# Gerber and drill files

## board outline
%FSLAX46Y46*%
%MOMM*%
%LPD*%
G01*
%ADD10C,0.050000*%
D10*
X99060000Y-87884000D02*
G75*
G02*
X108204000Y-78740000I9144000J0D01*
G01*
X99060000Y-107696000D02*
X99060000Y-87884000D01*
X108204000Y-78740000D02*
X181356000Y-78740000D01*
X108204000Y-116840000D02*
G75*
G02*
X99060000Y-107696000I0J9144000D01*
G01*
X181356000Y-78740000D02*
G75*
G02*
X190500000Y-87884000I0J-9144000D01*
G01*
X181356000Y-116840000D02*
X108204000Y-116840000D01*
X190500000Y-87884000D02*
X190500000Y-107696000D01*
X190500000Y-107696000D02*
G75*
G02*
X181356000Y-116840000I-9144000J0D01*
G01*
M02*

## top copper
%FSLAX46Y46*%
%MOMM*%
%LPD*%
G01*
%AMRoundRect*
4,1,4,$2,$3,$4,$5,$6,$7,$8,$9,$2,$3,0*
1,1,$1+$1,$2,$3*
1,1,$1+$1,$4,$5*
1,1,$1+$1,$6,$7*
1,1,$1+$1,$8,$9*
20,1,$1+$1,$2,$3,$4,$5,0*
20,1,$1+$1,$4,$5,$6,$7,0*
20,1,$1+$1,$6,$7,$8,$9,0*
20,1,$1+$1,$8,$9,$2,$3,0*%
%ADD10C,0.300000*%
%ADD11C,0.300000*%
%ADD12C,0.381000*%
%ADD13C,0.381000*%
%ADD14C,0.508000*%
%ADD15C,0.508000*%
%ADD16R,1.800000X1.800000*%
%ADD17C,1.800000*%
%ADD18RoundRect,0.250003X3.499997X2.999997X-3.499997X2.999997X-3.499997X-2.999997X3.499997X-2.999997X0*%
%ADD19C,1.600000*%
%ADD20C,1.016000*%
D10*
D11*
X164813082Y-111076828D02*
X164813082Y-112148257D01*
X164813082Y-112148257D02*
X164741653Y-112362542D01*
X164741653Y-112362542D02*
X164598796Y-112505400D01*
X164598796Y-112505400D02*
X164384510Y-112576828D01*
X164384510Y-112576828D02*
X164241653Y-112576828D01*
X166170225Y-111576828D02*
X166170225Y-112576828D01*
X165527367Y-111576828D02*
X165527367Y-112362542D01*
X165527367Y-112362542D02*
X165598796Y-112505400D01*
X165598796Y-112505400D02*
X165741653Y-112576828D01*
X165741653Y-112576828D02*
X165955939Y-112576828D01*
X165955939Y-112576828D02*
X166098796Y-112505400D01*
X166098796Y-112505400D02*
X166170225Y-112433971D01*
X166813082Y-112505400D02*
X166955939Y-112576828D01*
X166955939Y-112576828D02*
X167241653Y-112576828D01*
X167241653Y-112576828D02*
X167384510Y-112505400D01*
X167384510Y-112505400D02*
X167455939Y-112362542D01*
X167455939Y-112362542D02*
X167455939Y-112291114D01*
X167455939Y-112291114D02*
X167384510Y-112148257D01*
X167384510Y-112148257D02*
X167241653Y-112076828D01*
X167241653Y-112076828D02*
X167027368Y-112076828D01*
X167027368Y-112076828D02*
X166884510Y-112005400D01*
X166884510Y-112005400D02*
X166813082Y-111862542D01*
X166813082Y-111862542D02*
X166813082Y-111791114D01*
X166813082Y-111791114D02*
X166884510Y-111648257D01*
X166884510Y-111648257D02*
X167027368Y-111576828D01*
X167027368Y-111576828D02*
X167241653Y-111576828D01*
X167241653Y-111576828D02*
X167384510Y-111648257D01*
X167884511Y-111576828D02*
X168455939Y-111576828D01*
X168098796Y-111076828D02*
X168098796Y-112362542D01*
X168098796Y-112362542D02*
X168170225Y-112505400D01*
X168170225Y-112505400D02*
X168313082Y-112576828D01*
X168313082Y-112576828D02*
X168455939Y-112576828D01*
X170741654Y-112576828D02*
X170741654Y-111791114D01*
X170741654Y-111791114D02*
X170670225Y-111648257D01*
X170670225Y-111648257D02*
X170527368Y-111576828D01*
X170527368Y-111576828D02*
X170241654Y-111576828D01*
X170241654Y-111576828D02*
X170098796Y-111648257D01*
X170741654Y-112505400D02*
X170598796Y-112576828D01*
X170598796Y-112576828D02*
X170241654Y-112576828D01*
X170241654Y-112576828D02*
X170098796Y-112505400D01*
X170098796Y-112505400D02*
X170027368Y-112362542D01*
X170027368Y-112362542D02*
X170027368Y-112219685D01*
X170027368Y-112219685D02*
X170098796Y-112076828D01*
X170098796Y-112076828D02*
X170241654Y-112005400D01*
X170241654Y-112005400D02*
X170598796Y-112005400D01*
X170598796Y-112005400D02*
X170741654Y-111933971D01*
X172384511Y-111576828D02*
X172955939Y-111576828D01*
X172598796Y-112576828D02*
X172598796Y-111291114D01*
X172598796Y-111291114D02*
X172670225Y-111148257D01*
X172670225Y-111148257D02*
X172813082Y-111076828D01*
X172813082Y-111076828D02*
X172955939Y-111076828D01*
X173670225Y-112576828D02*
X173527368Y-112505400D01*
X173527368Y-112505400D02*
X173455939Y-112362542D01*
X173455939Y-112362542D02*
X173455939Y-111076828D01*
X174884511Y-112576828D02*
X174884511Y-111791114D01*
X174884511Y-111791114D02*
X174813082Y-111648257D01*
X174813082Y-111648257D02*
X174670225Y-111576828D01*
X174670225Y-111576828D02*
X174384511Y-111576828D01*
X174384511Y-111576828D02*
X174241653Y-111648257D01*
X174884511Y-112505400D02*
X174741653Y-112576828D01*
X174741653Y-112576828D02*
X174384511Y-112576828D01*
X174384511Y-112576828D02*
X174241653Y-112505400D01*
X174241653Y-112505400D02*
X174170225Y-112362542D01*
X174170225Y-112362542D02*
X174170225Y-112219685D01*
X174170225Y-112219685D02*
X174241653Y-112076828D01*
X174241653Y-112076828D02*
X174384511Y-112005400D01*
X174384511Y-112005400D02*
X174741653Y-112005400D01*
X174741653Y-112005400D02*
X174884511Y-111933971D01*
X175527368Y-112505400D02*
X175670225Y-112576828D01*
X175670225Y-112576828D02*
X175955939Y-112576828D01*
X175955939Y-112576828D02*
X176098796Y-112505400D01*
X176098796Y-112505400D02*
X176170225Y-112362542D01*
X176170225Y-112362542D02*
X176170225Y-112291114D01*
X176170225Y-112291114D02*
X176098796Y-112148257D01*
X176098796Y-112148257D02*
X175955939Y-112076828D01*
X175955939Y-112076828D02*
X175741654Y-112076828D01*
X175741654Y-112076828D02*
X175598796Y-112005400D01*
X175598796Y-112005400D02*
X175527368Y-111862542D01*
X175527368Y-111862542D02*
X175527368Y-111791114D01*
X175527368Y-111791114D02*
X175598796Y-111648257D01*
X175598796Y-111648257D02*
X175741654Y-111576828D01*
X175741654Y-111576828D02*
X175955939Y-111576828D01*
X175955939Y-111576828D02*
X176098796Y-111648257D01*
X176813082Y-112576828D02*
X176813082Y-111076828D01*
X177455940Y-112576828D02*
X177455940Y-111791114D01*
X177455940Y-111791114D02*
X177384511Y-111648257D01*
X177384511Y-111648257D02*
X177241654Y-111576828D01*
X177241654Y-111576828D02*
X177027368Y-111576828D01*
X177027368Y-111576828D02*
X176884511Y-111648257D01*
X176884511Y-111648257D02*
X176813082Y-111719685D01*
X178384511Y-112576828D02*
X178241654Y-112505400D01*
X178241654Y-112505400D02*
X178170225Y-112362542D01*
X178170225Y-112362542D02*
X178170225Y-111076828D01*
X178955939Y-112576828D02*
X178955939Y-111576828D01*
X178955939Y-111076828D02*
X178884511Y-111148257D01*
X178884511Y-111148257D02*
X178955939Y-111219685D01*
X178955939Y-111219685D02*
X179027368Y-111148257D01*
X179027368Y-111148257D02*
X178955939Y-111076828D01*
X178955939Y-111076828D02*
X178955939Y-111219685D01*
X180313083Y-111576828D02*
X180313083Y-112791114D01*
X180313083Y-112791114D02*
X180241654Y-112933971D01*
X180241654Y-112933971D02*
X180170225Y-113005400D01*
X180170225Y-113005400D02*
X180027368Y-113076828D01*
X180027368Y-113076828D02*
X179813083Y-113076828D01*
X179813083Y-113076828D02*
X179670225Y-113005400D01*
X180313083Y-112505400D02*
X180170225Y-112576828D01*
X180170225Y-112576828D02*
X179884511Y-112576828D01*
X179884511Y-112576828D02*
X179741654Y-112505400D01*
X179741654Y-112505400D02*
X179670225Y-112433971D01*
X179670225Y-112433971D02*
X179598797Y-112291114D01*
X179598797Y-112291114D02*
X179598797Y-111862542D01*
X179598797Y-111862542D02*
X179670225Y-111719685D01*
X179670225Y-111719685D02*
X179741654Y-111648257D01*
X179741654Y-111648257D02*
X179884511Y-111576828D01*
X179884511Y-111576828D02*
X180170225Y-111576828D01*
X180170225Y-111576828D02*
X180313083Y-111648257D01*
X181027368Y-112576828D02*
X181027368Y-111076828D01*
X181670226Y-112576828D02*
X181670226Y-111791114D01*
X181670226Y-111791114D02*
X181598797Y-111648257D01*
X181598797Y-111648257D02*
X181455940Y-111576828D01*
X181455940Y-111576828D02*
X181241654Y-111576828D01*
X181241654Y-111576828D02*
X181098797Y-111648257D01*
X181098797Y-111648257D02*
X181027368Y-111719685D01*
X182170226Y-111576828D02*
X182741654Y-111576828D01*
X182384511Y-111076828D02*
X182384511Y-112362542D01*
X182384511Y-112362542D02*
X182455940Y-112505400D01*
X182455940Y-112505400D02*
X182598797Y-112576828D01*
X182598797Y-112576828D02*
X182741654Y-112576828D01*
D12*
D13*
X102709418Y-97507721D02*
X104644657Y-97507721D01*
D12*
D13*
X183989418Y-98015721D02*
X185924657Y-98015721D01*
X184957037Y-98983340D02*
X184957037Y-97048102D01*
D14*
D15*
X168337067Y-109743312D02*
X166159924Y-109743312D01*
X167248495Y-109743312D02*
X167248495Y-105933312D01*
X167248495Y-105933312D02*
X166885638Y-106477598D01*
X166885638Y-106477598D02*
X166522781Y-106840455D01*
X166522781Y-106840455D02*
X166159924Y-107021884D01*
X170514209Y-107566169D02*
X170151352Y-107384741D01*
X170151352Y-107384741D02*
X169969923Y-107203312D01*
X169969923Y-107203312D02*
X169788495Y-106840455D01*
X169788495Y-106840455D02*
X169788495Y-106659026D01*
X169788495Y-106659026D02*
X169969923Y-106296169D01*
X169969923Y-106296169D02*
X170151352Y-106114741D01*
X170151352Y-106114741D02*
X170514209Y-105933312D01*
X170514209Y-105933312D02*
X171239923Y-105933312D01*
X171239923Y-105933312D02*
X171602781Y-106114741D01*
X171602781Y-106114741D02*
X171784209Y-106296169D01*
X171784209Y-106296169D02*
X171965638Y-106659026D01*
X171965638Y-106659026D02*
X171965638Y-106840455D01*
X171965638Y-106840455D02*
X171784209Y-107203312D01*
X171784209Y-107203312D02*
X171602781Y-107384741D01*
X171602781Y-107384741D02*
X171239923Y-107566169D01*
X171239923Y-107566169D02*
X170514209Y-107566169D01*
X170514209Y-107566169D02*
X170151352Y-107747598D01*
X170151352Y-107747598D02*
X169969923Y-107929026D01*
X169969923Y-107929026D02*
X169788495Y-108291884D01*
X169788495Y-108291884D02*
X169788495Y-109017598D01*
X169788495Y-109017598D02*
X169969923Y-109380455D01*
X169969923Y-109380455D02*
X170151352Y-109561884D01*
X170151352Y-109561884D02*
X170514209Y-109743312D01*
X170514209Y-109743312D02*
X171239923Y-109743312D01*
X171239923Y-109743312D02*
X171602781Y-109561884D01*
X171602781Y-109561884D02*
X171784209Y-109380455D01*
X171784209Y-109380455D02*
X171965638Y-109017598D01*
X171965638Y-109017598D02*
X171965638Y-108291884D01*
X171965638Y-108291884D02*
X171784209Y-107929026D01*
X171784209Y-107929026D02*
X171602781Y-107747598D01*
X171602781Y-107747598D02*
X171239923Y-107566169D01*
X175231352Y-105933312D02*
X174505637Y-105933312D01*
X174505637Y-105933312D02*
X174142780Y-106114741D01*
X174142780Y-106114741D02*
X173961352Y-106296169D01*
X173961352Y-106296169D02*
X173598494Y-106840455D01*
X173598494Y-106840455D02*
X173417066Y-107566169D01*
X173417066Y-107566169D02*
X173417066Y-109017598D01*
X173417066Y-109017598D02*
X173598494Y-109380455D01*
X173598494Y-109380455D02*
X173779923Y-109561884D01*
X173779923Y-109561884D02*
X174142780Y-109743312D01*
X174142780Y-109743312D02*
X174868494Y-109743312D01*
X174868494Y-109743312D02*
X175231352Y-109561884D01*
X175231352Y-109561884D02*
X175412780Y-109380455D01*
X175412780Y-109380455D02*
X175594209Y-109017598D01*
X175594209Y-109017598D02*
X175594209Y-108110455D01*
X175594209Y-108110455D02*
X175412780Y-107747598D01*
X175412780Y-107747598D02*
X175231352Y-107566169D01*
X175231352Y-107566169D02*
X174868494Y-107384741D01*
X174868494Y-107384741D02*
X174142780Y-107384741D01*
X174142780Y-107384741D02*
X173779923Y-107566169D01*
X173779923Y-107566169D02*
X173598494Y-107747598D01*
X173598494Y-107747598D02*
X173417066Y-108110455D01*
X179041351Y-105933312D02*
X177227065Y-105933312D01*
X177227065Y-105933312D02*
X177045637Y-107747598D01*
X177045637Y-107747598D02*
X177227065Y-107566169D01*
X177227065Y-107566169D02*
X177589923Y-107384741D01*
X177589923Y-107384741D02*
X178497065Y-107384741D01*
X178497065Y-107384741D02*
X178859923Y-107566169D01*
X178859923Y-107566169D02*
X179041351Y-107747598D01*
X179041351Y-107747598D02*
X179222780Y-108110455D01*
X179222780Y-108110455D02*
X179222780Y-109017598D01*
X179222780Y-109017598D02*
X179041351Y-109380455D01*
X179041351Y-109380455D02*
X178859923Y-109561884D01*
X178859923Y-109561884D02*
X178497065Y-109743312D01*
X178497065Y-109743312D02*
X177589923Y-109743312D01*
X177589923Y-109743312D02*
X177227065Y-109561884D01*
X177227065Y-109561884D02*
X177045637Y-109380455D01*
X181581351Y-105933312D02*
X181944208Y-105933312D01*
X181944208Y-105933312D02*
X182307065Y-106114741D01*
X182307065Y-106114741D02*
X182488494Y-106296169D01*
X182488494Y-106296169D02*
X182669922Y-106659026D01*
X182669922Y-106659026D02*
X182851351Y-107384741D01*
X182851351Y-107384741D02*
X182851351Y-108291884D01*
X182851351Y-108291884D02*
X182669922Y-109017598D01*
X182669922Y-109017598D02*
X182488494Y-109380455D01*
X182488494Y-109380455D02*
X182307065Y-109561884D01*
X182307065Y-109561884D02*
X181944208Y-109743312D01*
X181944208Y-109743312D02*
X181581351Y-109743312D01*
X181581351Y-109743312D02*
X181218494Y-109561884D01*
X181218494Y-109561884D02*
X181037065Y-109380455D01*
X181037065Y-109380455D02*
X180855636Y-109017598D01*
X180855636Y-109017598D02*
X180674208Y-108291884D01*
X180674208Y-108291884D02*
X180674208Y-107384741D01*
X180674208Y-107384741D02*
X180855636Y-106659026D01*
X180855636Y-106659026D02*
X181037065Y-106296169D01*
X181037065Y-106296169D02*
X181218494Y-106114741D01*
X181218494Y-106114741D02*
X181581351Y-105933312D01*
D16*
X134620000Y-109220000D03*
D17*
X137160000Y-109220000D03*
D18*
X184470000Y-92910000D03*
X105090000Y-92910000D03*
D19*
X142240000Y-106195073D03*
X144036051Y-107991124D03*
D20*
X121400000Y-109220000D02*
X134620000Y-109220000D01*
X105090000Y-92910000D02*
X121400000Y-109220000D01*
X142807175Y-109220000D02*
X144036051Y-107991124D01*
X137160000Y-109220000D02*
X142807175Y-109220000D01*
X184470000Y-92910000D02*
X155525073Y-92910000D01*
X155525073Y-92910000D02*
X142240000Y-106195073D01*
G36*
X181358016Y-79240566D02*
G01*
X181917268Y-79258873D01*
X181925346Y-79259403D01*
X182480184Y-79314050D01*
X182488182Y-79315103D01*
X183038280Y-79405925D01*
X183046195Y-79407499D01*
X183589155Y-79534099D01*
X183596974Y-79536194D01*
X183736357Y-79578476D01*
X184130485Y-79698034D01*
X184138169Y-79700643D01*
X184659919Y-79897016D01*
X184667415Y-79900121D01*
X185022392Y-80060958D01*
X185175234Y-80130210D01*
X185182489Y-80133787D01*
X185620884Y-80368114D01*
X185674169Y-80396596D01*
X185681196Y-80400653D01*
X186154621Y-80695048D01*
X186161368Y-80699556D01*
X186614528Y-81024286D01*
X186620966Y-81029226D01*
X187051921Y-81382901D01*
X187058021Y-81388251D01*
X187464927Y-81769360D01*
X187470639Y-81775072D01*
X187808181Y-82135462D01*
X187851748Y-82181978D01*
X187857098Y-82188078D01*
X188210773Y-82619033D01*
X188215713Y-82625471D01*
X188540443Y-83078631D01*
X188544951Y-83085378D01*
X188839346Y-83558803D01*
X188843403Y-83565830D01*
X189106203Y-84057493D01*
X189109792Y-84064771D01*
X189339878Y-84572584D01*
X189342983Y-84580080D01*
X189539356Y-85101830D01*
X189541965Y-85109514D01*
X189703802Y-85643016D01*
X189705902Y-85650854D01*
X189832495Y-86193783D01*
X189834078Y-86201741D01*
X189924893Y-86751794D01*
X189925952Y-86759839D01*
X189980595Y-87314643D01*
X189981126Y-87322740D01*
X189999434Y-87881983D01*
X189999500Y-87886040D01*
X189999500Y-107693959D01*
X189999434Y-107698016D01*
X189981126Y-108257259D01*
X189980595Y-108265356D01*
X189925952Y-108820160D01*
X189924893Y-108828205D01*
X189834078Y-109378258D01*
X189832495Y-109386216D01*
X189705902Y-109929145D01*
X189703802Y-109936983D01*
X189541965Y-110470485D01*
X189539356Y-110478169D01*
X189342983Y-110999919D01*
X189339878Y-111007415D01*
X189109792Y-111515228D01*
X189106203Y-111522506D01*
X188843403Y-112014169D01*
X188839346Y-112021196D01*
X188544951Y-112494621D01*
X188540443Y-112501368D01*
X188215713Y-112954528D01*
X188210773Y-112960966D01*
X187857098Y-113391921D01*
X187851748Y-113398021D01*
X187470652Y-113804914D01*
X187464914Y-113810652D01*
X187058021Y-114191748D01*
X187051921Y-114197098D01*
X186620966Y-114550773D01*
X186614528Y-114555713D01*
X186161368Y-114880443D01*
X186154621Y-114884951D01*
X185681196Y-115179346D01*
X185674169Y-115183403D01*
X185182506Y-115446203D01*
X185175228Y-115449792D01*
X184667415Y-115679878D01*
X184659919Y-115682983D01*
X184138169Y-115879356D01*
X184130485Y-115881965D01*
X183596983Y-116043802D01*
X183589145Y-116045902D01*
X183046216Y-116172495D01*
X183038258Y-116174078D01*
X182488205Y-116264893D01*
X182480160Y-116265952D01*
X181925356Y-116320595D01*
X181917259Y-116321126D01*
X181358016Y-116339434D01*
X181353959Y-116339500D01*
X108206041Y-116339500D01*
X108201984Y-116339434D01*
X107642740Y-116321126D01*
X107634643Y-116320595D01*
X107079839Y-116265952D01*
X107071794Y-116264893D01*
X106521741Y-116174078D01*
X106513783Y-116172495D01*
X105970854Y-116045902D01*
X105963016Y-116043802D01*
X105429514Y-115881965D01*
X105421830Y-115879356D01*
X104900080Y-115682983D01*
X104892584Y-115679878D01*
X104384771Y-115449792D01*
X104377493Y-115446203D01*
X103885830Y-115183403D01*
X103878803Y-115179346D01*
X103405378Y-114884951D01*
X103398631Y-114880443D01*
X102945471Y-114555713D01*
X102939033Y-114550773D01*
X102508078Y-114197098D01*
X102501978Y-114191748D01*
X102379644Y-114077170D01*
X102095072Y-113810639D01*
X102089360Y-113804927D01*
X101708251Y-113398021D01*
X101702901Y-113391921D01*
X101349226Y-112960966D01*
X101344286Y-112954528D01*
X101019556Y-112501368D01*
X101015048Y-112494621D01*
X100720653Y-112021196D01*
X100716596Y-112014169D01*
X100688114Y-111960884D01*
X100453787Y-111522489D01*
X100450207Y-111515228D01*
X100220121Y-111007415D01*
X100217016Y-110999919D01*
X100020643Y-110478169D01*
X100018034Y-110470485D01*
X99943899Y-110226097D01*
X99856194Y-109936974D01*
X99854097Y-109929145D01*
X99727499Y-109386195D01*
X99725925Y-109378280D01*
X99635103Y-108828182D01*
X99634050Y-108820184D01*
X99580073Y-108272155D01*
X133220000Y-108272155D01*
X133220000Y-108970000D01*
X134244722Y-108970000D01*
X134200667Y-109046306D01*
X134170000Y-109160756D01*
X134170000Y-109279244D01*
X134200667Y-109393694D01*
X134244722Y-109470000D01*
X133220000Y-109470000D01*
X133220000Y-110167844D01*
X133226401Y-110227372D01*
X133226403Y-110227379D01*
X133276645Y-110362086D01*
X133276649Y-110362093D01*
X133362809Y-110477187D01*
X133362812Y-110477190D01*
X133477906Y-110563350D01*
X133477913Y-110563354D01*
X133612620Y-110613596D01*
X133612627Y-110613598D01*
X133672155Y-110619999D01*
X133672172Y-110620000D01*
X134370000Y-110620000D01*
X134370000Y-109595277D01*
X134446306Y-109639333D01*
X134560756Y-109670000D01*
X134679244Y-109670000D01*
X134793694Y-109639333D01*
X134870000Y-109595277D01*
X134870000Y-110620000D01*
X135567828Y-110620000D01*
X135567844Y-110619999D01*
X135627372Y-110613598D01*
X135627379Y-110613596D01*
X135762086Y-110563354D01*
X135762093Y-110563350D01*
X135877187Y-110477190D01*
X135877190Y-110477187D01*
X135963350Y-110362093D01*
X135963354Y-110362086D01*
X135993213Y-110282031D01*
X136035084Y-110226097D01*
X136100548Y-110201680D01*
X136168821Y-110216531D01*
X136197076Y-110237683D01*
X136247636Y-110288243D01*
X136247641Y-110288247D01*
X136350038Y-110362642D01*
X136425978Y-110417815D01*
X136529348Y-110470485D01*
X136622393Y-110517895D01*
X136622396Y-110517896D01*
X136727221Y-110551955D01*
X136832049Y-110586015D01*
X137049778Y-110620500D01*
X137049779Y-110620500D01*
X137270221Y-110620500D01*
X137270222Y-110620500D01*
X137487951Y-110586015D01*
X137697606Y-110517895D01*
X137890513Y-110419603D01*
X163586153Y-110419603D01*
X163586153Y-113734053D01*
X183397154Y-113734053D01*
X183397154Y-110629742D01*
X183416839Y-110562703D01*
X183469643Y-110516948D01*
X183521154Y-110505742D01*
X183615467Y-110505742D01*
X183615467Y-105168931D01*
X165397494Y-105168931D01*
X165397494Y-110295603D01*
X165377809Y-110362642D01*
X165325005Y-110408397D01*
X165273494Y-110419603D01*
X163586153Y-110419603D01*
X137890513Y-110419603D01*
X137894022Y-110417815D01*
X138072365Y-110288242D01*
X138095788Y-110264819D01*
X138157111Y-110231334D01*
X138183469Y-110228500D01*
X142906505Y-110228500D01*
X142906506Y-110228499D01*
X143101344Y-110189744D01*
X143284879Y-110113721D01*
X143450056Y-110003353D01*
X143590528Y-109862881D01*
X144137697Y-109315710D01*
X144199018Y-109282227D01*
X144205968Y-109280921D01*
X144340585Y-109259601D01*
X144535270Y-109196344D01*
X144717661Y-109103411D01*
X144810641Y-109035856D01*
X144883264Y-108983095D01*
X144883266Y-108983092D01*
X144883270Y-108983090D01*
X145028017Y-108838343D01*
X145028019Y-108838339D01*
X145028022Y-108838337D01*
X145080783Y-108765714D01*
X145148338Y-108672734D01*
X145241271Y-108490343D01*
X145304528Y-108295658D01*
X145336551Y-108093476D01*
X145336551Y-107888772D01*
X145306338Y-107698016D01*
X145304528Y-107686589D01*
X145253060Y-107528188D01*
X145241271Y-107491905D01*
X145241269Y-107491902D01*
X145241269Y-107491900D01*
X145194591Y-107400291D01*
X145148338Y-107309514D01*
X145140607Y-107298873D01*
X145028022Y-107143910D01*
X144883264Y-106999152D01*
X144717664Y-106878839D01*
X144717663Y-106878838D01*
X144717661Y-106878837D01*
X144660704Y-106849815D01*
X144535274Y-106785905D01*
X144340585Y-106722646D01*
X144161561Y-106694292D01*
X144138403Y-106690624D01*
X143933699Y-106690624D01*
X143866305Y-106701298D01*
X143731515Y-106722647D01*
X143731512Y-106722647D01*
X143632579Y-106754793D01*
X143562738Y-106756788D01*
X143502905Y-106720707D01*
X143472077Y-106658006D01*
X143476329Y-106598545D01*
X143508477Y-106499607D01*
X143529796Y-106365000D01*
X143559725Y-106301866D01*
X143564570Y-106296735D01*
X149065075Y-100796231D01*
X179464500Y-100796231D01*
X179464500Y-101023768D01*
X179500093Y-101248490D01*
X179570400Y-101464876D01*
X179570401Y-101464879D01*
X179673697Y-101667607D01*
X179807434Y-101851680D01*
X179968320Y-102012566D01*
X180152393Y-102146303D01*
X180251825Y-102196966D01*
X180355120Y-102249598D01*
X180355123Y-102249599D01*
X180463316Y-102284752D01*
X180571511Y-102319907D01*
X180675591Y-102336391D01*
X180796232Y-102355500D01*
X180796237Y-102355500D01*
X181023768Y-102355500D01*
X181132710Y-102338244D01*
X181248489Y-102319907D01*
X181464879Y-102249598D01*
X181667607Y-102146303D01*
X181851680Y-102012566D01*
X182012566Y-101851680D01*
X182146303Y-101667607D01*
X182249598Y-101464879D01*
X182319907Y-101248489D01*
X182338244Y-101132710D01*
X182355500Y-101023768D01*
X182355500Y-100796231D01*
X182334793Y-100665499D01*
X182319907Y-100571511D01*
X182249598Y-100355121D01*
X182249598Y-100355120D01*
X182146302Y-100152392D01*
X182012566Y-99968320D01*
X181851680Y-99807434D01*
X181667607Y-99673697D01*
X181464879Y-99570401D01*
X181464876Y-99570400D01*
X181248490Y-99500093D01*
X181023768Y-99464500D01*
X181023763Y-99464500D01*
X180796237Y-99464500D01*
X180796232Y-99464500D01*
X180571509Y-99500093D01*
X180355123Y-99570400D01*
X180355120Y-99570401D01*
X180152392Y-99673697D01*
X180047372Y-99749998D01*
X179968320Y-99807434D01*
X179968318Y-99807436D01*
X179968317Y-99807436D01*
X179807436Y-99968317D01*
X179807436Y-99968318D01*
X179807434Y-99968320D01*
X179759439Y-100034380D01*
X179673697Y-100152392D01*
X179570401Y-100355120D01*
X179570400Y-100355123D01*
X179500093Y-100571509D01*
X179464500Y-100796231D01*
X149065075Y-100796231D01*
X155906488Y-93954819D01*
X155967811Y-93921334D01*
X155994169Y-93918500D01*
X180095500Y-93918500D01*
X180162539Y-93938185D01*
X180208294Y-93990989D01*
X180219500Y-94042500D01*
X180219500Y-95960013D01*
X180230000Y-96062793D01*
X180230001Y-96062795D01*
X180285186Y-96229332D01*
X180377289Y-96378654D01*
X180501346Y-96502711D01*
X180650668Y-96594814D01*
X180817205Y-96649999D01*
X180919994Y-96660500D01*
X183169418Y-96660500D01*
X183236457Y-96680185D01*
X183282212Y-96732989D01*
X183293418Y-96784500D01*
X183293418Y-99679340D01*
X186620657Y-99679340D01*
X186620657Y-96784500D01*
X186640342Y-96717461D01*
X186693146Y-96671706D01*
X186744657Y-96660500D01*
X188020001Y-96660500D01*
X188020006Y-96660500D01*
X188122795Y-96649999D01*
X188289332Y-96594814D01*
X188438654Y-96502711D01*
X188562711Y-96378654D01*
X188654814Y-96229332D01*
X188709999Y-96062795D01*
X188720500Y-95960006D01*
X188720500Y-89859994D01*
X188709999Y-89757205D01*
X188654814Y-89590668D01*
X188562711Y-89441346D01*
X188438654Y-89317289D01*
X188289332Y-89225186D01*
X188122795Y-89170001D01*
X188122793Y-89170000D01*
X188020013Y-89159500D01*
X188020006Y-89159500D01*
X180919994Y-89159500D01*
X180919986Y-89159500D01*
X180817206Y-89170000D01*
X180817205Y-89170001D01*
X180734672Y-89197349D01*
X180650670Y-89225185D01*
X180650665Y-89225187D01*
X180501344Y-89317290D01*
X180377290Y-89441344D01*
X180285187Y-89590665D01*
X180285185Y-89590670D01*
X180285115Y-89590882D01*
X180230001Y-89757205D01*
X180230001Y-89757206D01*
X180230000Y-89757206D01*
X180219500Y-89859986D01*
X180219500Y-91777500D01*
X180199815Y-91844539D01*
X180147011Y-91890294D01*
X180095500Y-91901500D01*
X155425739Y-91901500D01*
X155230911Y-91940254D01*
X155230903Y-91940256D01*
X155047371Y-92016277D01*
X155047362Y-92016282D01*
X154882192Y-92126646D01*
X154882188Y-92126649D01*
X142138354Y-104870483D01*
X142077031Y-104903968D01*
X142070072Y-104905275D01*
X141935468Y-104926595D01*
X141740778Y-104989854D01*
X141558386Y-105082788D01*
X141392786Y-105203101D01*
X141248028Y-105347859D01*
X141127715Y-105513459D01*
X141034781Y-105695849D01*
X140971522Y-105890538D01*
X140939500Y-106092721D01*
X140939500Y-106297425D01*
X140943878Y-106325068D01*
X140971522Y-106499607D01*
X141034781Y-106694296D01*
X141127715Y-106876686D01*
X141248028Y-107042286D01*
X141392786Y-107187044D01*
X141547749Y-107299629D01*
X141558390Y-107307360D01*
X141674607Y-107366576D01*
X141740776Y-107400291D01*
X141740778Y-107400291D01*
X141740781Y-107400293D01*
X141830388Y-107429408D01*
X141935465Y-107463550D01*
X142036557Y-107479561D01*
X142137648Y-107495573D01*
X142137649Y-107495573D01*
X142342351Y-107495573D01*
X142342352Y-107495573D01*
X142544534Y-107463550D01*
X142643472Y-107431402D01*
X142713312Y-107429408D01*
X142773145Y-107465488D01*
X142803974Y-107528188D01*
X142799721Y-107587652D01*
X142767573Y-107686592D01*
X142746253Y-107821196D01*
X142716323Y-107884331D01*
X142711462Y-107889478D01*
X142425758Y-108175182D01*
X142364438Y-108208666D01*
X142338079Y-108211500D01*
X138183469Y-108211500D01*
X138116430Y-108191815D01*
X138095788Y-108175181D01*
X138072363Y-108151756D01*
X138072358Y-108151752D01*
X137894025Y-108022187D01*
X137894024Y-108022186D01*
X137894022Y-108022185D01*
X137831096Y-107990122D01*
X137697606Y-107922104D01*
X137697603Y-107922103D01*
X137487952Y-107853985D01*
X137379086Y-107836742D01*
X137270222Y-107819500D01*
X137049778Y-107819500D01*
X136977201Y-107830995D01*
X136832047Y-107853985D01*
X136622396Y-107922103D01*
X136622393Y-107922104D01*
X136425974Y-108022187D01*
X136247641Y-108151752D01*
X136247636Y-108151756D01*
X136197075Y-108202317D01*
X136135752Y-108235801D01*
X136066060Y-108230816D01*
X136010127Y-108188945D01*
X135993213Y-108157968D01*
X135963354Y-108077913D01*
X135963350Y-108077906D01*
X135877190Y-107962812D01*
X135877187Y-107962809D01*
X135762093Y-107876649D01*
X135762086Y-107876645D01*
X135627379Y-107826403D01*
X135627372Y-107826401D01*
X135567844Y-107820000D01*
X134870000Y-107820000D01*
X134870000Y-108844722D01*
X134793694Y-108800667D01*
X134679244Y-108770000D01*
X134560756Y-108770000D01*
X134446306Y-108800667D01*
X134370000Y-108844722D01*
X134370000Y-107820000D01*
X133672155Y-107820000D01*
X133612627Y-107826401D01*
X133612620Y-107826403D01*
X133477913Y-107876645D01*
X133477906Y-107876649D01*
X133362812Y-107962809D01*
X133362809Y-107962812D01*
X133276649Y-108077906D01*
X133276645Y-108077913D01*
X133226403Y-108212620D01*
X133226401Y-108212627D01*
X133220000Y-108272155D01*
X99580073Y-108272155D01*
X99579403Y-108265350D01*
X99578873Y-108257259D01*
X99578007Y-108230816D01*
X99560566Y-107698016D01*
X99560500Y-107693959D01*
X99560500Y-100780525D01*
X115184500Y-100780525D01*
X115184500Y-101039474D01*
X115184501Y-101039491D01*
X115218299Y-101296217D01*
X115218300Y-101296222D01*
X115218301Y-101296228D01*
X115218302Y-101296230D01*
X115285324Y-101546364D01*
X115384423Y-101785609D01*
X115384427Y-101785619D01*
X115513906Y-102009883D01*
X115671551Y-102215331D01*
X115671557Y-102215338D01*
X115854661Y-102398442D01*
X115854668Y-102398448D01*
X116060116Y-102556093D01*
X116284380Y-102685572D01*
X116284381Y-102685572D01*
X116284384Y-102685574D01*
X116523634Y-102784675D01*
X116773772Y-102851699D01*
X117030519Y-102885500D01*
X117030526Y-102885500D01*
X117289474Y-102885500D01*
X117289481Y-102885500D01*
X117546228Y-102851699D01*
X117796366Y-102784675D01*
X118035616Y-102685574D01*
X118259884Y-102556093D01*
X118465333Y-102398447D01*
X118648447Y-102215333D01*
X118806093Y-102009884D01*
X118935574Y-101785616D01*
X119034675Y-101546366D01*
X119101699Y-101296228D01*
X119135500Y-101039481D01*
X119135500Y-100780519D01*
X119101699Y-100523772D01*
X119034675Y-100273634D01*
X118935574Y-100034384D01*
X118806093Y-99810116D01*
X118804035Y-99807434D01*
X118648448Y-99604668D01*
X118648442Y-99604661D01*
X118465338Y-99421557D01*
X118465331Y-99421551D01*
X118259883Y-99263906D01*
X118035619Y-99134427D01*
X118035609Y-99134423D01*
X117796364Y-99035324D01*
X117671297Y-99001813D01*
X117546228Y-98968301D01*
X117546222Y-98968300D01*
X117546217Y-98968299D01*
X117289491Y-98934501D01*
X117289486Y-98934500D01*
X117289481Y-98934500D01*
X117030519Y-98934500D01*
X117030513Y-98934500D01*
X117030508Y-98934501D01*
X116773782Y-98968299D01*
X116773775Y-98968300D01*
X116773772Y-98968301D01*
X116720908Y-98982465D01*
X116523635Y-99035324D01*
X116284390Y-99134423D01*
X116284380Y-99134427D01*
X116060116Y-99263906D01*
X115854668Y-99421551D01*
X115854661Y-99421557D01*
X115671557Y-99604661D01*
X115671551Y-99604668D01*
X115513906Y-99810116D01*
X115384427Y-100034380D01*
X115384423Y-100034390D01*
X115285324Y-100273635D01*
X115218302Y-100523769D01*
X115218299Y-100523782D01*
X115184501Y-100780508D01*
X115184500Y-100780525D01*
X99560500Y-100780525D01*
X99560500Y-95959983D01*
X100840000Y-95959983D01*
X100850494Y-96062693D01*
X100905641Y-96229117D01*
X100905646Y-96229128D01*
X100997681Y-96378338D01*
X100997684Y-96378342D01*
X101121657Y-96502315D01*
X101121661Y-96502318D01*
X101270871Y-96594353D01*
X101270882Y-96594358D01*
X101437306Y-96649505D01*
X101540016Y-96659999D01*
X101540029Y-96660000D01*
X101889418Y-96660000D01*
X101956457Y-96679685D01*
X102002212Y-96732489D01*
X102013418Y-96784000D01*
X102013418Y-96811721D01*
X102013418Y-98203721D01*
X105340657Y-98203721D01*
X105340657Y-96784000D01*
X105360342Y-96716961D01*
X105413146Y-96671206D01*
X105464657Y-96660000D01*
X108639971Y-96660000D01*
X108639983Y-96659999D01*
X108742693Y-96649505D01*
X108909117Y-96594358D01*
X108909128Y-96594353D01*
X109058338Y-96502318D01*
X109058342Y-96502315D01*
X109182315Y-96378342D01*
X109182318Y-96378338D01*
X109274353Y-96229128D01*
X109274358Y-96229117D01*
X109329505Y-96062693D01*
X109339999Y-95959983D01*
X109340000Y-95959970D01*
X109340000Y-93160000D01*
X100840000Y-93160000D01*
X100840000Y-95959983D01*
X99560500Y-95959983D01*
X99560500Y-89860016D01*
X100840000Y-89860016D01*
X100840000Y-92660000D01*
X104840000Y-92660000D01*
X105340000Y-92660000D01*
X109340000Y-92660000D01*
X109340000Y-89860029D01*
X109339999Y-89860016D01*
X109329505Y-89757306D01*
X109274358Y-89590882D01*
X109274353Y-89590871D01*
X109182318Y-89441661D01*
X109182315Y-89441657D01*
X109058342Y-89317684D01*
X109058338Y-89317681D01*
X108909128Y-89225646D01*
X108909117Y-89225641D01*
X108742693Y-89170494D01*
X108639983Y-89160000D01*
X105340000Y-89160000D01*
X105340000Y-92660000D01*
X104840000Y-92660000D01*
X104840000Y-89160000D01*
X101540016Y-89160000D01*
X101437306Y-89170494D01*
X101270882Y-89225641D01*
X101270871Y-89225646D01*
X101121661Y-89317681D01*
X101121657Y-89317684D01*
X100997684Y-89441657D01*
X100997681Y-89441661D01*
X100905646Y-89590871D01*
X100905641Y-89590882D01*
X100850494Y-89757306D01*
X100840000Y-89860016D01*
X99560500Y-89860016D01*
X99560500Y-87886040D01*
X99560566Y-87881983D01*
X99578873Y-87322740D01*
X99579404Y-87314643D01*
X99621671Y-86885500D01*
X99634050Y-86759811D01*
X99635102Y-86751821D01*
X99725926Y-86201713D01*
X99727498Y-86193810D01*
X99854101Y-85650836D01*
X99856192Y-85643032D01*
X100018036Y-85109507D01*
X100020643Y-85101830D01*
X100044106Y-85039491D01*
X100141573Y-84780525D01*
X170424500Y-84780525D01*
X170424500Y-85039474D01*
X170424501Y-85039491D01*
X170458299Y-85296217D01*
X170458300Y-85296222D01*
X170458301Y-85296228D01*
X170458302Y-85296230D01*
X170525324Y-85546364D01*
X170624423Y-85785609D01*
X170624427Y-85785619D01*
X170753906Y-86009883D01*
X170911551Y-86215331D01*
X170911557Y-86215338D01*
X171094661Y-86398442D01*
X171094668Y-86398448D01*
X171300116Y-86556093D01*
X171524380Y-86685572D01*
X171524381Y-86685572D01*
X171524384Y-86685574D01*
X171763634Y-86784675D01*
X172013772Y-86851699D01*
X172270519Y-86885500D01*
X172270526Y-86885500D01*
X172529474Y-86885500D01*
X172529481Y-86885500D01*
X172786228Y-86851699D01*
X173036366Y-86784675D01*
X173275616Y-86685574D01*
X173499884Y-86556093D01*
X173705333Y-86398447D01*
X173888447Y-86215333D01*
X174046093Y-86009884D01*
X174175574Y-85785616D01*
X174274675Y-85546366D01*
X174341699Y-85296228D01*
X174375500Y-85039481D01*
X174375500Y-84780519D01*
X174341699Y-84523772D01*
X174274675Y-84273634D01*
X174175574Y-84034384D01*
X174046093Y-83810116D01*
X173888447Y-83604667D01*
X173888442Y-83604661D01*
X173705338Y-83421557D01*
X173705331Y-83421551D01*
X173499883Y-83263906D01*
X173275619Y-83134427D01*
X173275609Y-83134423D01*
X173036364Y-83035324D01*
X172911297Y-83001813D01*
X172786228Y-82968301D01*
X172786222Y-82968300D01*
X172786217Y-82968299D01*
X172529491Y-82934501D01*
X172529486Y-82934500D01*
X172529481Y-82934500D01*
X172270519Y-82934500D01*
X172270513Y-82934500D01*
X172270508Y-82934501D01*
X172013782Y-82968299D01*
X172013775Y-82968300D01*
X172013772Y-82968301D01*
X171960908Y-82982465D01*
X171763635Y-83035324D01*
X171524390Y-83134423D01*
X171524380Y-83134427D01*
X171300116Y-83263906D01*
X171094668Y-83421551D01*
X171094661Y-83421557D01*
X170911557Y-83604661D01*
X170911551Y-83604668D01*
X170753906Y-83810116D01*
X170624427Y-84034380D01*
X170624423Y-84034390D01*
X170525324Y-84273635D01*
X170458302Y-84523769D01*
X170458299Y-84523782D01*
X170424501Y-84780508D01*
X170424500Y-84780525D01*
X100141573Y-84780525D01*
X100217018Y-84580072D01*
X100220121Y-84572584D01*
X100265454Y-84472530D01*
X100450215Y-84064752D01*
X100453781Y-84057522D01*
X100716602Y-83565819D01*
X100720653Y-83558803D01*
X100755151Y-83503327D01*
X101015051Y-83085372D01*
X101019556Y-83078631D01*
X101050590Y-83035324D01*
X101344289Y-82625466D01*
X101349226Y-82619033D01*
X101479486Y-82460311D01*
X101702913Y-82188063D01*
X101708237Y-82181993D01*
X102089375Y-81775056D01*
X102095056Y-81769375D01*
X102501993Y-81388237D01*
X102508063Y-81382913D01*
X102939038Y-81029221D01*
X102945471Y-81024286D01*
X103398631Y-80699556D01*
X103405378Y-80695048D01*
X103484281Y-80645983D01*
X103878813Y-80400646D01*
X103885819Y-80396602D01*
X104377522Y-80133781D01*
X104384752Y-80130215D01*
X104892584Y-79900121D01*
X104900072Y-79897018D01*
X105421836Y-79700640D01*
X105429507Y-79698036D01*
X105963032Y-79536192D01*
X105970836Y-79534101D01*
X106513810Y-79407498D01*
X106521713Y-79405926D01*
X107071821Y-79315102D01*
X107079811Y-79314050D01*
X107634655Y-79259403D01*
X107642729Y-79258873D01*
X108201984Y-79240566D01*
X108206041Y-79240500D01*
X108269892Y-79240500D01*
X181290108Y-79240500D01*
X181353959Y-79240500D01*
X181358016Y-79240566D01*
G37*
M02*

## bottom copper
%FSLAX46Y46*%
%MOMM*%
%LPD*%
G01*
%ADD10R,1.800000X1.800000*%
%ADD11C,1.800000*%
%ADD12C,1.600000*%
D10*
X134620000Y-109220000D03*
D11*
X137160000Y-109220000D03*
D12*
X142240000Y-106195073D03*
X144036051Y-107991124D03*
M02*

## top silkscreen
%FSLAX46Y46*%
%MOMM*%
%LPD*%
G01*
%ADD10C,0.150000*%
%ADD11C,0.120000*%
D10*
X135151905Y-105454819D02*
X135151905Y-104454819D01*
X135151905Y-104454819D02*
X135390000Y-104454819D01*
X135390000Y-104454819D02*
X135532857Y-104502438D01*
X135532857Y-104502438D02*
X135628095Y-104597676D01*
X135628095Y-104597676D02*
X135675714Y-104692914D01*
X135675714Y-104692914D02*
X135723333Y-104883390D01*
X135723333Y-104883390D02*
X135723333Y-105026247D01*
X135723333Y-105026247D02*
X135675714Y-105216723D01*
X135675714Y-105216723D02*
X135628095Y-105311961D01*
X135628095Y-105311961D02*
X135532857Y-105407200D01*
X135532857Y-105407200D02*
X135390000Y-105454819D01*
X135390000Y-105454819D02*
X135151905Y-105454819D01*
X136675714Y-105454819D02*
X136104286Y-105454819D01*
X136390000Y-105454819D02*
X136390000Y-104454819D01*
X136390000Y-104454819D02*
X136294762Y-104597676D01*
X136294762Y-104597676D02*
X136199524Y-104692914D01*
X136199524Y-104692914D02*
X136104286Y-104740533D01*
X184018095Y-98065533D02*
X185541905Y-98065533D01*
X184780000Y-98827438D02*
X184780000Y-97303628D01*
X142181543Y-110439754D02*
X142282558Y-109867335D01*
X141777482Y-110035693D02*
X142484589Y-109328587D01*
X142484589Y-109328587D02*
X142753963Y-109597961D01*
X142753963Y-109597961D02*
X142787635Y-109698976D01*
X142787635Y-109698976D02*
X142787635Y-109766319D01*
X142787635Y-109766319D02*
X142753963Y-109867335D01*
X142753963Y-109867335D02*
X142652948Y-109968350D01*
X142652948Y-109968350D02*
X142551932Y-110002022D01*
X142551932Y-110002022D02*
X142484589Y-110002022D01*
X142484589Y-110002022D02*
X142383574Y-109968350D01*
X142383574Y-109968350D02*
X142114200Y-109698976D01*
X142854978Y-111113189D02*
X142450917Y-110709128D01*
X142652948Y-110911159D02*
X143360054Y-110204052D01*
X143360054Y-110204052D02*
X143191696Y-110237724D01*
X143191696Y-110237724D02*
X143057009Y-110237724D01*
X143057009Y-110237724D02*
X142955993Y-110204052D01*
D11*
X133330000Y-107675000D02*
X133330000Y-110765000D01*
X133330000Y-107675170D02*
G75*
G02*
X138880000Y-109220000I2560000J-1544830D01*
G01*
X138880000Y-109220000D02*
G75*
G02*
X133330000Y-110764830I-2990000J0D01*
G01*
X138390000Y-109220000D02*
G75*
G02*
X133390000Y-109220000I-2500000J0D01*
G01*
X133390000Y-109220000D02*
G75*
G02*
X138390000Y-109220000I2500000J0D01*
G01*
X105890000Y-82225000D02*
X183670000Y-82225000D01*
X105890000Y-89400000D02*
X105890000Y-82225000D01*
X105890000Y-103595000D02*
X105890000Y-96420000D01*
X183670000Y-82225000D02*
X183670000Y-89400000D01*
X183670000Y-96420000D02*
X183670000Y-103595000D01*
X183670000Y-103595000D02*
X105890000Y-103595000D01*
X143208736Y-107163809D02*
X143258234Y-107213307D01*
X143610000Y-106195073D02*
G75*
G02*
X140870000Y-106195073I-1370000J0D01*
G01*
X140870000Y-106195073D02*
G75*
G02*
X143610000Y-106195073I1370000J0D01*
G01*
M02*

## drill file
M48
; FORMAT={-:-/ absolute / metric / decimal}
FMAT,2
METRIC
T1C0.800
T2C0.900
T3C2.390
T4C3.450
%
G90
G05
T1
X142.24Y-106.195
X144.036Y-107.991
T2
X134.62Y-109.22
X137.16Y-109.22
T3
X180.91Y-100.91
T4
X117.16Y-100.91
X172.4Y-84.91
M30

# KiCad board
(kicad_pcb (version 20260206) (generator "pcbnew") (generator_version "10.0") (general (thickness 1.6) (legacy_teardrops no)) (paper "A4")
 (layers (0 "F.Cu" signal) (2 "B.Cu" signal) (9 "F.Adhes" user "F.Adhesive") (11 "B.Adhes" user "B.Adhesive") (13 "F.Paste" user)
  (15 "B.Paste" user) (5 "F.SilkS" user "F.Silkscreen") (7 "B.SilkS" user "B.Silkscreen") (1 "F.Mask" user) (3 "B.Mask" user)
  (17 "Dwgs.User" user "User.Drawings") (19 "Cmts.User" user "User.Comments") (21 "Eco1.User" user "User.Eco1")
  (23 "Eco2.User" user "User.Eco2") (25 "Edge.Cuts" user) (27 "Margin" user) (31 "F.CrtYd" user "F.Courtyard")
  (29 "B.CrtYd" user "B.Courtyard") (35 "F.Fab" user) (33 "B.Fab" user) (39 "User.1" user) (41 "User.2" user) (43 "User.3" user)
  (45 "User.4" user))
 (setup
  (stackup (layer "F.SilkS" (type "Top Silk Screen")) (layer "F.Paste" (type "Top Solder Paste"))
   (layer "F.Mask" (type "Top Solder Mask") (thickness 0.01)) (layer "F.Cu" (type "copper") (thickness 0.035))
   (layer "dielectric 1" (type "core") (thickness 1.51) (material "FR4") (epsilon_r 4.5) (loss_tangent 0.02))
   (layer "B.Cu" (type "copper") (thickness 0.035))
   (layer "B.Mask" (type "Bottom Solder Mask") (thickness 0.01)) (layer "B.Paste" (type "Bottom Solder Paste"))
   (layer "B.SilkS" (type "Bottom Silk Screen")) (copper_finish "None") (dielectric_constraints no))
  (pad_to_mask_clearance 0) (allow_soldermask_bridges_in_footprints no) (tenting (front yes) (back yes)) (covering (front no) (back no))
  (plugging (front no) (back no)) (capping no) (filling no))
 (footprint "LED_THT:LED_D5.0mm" (layer "F.Cu") (at 134.62 109.22)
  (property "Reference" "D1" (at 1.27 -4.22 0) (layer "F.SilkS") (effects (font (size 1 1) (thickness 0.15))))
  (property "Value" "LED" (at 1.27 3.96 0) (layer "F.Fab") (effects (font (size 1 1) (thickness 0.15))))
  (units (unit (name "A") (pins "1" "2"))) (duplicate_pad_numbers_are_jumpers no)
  (fp_line (start -1.29 -1.545) (end -1.29 1.545) (stroke (width 0.12) (type solid)) (layer "F.SilkS"))
  (fp_arc (start -1.29 -1.54483) (mid 2.071779 -2.880495) (end 4.26 0) (stroke (width 0.12) (type solid)) (layer "F.SilkS"))
  (fp_arc (start 4.26 0) (mid 2.071779 2.880495) (end -1.29 1.54483) (stroke (width 0.12) (type solid)) (layer "F.SilkS"))
  (fp_circle (center 1.27 0) (end 3.77 0) (stroke (width 0.12) (type solid)) (fill no) (layer "F.SilkS"))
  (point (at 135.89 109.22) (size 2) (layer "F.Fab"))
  (pad "1" thru_hole rect (at 0 0) (size 1.8 1.8) (drill 0.9) (layers "*.Cu" "*.Mask") (remove_unused_layers no) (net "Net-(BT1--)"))
  (pad "2" thru_hole circle (at 2.54 0) (size 1.8 1.8) (drill 0.9) (layers "*.Cu" "*.Mask") (remove_unused_layers no) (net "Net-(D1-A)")))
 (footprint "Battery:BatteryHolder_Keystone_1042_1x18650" (layer "F.Cu") (at 144.78 92.91 180)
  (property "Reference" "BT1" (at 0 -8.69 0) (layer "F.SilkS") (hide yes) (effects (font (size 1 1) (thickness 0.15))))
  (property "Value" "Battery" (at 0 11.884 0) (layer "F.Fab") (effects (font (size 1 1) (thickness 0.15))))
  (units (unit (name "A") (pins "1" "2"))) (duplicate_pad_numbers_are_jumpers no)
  (fp_line (start 38.89 10.685) (end -38.89 10.685) (stroke (width 0.12) (type solid)) (layer "F.SilkS"))
  (fp_line (start 38.89 3.51) (end 38.89 10.685) (stroke (width 0.12) (type solid)) (layer "F.SilkS"))
  (fp_line (start 38.89 -10.685) (end 38.89 -3.51) (stroke (width 0.12) (type solid)) (layer "F.SilkS"))
  (fp_line (start -38.89 10.685) (end -38.89 3.51) (stroke (width 0.12) (type solid)) (layer "F.SilkS"))
  (fp_line (start -38.89 -3.51) (end -38.89 -10.685) (stroke (width 0.12) (type solid)) (layer "F.SilkS"))
  (fp_line (start -38.89 -10.685) (end 38.89 -10.685) (stroke (width 0.12) (type solid)) (layer "F.SilkS"))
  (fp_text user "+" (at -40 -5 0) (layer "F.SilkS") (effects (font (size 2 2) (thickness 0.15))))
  (pad "" np_thru_hole circle (at -36.13 -8 180) (size 2.39 2.39) (drill 2.39) (layers "*.Cu" "*.Mask"))
  (pad "" np_thru_hole circle (at -27.62 8 180) (size 3.45 3.45) (drill 3.45) (layers "*.Cu" "*.Mask"))
  (pad "" np_thru_hole circle (at 27.62 -8 180) (size 3.45 3.45) (drill 3.45) (layers "*.Cu" "*.Mask"))
  (pad "1" smd roundrect (at -39.69 0 180) (size 7.5 6.5) (layers "F.Cu" "F.Mask" "F.Paste") (roundrect_rratio 0.038462) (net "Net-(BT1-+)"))
  (pad "2" smd roundrect (at 39.69 0 180) (size 7.5 6.5) (layers "F.Cu" "F.Mask" "F.Paste") (roundrect_rratio 0.038462) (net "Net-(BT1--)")))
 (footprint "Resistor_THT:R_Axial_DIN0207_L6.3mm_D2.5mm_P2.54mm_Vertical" (layer "F.Cu") (at 142.24 106.195073 -45)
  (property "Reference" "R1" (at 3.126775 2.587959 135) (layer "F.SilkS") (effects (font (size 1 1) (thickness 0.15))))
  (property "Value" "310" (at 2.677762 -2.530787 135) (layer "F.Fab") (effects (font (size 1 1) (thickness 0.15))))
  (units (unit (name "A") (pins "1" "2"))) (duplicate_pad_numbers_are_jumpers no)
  (fp_line (start 1.37 0) (end 1.44 0) (stroke (width 0.12) (type solid)) (layer "F.SilkS"))
  (fp_circle (center 0 0) (end 1.37 0) (stroke (width 0.12) (type solid)) (fill no) (layer "F.SilkS"))
  (pad "1" thru_hole circle (at 0 0 315) (size 1.6 1.6) (drill 0.8) (layers "*.Cu" "*.Mask") (remove_unused_layers no) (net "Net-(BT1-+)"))
  (pad "2" thru_hole circle (at 2.54 0 315) (size 1.6 1.6) (drill 0.8) (layers "*.Cu" "*.Mask") (remove_unused_layers no) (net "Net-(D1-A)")))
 (gr_arc (start 99.06 87.884) (mid 101.738216 81.418216) (end 108.204 78.74) (stroke (width 0.05) (type default)) (layer "Edge.Cuts"))
 (gr_line (start 99.06 107.696) (end 99.06 87.884) (stroke (width 0.05) (type default)) (layer "Edge.Cuts"))
 (gr_line (start 108.204 78.74) (end 181.356 78.74) (stroke (width 0.05) (type default)) (layer "Edge.Cuts"))
 (gr_arc (start 108.204 116.84) (mid 101.738216 114.161784) (end 99.06 107.696) (stroke (width 0.05) (type default)) (layer "Edge.Cuts"))
 (gr_arc (start 181.356 78.74) (mid 187.821784 81.418216) (end 190.5 87.884) (stroke (width 0.05) (type default)) (layer "Edge.Cuts"))
 (gr_line (start 181.356 116.84) (end 108.204 116.84) (stroke (width 0.05) (type default)) (layer "Edge.Cuts"))
 (gr_line (start 190.5 87.884) (end 190.5 107.696) (stroke (width 0.05) (type default)) (layer "Edge.Cuts"))
 (gr_arc (start 190.5 107.696) (mid 187.821784 114.161784) (end 181.356 116.84) (stroke (width 0.05) (type default)) (layer "Edge.Cuts"))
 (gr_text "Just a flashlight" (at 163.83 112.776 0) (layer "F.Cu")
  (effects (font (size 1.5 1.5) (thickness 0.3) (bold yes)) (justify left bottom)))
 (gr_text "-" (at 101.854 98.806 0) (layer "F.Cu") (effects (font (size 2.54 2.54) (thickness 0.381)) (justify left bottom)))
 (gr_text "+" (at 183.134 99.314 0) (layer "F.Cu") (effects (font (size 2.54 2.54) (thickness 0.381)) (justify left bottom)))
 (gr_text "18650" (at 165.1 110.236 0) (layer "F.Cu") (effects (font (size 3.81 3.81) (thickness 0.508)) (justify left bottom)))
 (segment (start 121.4 109.22) (end 134.62 109.22) (width 1.016) (layer "F.Cu") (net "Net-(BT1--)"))
 (segment (start 105.09 92.91) (end 121.4 109.22) (width 1.016) (layer "F.Cu") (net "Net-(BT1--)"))
 (segment (start 142.807175 109.22) (end 144.036051 107.991124) (width 1.016) (layer "F.Cu") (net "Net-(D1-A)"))
 (segment (start 137.16 109.22) (end 142.807175 109.22) (width 1.016) (layer "F.Cu") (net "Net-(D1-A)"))
 (segment (start 184.47 92.91) (end 155.525073 92.91) (width 1.016) (layer "F.Cu") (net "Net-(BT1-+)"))
 (segment (start 155.525073 92.91) (end 142.24 106.195073) (width 1.016) (layer "F.Cu") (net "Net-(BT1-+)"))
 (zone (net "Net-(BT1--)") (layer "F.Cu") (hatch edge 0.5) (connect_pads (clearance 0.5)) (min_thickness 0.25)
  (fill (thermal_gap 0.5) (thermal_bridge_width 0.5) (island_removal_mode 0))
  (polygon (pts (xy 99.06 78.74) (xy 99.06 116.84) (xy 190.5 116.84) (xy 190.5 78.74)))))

